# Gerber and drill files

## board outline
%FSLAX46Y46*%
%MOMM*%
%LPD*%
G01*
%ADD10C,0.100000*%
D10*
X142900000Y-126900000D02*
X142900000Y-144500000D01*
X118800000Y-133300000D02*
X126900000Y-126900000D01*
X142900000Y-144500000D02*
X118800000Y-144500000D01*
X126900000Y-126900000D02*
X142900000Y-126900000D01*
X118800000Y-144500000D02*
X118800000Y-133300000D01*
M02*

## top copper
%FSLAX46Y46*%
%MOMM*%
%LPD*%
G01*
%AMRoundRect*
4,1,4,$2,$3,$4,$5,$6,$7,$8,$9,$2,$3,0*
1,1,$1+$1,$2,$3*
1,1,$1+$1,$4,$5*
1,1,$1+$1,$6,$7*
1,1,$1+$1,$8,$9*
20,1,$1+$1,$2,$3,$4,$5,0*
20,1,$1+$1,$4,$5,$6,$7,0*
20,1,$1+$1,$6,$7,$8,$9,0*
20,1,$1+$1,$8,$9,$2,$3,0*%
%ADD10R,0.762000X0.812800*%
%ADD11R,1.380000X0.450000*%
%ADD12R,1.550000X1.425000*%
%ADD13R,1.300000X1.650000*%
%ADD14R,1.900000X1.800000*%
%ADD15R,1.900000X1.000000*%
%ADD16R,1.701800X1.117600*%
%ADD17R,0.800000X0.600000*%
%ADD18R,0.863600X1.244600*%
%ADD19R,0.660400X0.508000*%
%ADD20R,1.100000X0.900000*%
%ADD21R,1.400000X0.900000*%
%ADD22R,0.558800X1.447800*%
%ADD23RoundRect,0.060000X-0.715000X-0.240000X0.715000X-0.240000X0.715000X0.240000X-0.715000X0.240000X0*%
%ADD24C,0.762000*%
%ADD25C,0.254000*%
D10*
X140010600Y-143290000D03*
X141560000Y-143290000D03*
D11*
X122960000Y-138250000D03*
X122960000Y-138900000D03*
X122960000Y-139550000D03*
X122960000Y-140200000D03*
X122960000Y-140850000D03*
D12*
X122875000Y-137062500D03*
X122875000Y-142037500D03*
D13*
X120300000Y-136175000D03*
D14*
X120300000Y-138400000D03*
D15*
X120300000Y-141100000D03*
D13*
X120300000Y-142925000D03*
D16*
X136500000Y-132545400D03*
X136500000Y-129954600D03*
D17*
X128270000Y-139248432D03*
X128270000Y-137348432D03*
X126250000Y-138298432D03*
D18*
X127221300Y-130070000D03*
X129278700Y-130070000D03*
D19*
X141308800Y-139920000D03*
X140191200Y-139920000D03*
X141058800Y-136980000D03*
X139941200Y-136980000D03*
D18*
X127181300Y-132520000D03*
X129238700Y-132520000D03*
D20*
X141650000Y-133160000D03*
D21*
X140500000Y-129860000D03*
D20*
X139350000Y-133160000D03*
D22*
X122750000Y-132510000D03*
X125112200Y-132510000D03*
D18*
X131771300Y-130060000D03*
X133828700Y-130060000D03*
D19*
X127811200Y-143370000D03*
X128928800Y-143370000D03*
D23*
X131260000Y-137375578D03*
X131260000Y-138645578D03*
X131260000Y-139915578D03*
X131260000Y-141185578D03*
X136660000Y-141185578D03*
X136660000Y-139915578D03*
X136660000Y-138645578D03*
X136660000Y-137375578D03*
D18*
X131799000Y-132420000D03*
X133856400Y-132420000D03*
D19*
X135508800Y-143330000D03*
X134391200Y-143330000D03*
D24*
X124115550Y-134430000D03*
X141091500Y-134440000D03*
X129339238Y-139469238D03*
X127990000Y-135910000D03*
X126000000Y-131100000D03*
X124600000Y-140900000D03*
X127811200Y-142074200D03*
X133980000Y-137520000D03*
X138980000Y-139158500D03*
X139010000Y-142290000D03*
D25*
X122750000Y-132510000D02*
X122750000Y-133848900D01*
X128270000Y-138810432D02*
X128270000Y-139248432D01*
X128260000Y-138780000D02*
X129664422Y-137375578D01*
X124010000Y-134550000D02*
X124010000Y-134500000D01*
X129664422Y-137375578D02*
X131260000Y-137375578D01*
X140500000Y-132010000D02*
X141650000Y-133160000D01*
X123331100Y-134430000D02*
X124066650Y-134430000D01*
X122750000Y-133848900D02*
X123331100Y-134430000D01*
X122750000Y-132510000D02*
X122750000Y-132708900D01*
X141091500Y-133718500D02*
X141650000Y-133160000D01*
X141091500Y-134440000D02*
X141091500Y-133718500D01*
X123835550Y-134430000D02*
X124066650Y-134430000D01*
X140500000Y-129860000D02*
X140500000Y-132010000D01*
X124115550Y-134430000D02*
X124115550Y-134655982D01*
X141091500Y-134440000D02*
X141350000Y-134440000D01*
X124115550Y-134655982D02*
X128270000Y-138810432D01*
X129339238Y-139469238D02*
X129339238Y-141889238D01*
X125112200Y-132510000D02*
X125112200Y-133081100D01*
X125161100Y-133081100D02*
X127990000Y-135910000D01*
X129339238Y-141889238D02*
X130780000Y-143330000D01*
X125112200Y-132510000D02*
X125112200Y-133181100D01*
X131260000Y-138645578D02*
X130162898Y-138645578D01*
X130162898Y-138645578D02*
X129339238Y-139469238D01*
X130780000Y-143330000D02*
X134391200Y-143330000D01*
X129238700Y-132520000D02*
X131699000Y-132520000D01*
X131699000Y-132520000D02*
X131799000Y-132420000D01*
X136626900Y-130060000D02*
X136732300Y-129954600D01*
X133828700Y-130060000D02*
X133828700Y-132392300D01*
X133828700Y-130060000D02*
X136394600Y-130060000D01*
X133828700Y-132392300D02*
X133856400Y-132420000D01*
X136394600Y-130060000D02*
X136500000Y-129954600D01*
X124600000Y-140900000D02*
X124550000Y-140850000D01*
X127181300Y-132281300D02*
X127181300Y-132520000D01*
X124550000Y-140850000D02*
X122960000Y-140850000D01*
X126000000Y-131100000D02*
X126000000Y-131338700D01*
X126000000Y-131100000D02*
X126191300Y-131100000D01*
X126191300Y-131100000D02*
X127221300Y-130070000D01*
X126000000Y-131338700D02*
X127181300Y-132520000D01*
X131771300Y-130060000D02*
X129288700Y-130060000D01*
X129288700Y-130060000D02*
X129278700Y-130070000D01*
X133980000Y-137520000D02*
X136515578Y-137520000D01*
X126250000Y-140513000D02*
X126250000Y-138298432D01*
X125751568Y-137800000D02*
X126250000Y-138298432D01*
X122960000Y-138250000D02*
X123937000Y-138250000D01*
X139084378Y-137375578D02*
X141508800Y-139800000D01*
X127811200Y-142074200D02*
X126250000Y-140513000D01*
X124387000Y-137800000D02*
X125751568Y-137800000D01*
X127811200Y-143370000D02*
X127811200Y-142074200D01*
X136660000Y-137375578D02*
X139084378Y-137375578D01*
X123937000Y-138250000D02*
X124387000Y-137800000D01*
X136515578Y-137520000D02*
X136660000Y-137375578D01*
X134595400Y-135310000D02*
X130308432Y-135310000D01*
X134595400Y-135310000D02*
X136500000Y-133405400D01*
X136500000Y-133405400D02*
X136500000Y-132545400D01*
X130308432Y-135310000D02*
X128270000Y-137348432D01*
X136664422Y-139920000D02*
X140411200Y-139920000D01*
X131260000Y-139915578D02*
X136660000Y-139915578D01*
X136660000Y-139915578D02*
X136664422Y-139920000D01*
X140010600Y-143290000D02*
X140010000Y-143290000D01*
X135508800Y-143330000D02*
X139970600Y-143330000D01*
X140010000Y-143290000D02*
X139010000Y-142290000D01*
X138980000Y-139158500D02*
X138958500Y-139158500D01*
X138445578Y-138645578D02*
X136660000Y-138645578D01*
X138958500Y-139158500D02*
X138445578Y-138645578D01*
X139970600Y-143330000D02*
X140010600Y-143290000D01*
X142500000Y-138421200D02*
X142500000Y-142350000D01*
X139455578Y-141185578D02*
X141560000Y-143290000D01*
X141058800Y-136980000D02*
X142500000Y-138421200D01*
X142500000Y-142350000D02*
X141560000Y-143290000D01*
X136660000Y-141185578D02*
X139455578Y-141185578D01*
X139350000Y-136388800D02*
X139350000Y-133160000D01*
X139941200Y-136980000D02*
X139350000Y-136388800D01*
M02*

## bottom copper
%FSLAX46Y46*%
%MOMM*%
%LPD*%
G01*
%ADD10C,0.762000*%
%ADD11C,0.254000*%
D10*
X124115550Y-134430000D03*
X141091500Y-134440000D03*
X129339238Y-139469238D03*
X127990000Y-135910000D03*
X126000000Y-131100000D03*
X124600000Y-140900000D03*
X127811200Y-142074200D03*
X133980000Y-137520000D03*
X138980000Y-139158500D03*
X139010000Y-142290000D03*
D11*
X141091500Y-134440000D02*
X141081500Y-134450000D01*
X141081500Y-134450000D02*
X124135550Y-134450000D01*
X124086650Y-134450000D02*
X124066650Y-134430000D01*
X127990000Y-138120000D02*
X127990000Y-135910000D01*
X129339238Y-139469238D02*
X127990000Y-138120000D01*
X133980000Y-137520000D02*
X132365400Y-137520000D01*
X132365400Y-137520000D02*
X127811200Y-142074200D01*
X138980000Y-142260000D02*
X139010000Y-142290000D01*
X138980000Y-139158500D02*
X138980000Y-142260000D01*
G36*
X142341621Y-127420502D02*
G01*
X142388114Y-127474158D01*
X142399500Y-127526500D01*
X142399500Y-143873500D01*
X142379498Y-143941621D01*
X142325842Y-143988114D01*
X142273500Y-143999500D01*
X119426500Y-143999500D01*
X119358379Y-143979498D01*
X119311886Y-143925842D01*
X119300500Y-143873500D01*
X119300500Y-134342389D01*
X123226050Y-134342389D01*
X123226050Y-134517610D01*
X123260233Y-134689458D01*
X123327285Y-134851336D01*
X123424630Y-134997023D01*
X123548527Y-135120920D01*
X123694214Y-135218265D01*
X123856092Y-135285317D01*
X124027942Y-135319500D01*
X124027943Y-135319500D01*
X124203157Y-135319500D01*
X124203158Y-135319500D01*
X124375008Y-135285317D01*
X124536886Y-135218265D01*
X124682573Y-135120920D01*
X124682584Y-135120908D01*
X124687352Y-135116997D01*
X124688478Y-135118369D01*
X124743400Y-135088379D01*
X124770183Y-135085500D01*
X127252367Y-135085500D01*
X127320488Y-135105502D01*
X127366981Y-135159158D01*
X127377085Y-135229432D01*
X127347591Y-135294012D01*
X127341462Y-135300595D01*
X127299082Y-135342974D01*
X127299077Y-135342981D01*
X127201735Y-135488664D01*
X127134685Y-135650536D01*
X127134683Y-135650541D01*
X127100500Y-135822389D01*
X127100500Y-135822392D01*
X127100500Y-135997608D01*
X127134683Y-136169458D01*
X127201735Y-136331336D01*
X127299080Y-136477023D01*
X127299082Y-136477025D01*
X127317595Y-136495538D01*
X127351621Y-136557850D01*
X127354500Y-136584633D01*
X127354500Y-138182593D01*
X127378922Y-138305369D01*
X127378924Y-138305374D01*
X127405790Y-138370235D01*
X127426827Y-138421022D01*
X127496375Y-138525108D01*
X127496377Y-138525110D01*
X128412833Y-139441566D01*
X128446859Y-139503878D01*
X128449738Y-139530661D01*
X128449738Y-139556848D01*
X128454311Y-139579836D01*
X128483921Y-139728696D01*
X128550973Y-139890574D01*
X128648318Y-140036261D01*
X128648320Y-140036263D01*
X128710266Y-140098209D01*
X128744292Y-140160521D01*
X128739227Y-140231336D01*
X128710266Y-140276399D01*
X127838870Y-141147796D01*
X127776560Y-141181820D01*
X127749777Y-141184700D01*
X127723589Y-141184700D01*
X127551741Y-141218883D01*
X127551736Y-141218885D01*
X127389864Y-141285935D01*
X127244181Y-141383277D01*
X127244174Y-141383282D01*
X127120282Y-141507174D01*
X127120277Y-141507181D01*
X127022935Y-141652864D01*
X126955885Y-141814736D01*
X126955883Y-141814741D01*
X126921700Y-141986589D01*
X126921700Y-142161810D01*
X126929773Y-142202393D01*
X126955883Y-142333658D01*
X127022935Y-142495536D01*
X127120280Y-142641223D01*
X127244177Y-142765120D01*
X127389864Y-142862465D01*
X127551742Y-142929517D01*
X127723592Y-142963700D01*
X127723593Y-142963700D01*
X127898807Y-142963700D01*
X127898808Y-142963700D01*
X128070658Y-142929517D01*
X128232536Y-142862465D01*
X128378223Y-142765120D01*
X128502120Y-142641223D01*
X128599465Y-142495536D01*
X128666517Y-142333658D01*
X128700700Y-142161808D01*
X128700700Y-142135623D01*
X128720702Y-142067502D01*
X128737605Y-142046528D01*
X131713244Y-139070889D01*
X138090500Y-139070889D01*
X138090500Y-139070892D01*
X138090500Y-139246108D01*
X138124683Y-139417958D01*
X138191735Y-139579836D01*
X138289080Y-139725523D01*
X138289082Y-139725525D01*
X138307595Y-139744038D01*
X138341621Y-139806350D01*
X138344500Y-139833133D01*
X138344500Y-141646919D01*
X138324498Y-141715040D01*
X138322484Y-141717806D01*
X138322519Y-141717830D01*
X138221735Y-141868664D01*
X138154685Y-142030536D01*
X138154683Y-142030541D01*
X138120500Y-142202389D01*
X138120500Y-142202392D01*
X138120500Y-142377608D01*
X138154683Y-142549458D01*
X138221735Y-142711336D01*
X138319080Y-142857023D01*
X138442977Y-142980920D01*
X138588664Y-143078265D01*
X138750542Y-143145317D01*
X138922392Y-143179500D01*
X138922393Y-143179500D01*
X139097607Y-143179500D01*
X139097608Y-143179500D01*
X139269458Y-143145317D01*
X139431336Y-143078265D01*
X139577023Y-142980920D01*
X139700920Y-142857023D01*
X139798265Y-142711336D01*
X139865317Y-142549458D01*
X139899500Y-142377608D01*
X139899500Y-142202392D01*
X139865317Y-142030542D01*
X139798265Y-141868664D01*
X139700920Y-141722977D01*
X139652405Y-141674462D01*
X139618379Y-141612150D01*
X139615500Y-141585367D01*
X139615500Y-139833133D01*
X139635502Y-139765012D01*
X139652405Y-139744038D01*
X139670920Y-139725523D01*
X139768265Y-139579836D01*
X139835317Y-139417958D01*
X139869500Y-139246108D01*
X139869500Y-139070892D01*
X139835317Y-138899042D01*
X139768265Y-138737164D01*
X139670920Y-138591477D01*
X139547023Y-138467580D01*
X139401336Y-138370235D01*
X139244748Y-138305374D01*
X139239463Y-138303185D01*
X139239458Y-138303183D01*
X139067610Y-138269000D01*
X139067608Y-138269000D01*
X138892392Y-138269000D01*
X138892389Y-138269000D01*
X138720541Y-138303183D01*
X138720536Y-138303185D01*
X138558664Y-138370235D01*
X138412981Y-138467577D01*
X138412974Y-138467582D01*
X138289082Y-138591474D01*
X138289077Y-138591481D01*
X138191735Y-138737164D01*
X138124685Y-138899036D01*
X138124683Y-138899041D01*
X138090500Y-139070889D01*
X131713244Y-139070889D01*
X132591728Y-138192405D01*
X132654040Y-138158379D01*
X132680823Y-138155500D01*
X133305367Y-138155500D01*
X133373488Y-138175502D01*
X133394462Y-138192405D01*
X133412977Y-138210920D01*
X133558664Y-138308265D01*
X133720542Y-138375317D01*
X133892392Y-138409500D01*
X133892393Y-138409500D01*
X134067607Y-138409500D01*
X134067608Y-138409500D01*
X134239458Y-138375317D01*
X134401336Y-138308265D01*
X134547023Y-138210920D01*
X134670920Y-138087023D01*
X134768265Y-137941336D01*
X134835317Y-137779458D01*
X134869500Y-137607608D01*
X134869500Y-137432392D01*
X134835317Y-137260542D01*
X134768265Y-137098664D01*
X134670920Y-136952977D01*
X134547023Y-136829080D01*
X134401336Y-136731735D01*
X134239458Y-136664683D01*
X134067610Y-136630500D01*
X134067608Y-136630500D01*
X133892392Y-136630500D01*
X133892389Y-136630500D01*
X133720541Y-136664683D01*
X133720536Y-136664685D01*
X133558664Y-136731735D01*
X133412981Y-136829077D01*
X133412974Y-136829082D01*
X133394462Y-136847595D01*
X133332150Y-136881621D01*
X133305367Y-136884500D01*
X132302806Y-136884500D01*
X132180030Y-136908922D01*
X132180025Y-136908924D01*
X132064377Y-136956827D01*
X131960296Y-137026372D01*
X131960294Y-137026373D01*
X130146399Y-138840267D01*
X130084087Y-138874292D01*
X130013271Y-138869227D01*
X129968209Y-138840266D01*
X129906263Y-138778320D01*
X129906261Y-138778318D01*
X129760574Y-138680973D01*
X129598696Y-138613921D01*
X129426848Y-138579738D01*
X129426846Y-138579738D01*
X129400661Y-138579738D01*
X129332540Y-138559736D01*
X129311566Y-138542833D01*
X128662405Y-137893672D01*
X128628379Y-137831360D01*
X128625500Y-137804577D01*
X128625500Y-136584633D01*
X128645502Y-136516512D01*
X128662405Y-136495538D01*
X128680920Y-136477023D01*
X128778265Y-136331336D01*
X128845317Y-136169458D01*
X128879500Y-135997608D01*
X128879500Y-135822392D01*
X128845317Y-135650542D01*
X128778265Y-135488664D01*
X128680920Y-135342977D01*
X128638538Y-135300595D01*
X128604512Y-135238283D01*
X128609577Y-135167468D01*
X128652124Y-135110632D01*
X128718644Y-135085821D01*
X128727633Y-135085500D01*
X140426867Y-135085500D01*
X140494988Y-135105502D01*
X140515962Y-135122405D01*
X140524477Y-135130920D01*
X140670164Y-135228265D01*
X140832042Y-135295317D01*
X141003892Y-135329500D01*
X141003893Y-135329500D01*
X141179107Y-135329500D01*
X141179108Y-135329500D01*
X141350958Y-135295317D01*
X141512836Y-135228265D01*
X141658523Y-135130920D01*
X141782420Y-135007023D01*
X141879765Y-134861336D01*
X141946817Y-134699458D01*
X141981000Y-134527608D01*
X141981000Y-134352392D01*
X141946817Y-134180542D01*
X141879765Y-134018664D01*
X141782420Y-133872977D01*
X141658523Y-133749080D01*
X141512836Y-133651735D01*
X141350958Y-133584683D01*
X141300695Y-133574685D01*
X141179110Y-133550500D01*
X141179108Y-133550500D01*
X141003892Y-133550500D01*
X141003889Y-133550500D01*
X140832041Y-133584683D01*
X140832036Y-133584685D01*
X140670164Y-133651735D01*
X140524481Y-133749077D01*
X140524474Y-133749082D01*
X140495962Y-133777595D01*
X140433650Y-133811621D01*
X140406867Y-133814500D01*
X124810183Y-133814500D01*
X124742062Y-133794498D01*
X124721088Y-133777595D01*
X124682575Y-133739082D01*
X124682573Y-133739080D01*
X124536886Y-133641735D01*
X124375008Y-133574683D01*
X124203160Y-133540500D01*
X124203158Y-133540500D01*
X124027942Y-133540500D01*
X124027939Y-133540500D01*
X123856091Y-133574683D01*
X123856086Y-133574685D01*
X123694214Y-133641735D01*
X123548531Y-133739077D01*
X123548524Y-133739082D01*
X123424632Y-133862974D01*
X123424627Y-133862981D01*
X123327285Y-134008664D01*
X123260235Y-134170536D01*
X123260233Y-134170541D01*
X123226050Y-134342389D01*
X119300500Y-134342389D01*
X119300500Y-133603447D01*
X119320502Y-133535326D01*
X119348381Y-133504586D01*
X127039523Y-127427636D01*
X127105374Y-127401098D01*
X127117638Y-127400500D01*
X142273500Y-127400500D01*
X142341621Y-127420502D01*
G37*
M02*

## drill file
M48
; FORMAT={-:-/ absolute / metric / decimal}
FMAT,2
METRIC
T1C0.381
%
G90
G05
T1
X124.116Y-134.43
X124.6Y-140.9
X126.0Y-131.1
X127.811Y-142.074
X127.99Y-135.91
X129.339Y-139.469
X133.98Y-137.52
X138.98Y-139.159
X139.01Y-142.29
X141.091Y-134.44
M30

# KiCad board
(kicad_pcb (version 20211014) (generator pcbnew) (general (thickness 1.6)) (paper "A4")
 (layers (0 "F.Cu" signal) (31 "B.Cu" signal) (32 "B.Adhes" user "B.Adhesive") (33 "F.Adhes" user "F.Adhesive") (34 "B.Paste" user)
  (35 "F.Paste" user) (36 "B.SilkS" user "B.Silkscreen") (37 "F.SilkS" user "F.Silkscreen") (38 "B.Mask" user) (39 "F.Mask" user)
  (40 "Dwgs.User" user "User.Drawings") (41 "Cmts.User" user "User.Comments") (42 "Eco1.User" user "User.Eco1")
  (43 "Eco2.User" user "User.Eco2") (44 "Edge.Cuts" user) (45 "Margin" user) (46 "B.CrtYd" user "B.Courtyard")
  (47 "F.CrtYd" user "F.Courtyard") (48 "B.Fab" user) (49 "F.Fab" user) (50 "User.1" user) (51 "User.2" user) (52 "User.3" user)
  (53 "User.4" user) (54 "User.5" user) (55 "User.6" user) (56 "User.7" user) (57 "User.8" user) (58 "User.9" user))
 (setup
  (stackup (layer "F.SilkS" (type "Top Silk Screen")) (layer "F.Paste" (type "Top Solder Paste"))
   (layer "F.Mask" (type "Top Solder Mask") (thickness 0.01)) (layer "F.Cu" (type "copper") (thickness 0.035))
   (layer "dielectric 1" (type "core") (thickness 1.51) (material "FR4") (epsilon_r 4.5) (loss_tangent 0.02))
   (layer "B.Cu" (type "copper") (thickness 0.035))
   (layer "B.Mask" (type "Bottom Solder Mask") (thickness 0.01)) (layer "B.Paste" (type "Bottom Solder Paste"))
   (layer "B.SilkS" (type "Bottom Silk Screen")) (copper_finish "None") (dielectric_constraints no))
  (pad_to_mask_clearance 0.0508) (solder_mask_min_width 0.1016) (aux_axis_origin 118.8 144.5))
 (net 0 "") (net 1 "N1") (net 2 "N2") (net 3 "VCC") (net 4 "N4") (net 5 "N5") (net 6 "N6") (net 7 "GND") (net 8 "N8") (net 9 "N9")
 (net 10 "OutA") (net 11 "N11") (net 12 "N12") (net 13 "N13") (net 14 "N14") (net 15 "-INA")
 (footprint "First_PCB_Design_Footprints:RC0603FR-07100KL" (layer "F.Cu") (at 140.7853 143.29)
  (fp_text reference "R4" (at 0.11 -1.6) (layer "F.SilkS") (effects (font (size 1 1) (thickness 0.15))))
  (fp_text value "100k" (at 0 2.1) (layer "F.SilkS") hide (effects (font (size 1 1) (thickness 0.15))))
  (pad "1" smd rect (at -0.7747 0) (size 0.762 0.8128) (layers "F.Cu" "F.Paste" "F.Mask") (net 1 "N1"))
  (pad "2" smd rect (at 0.7747 0) (size 0.762 0.8128) (layers "F.Cu" "F.Paste" "F.Mask") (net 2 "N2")))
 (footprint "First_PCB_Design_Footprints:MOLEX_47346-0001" (layer "F.Cu") (at 120.3 139.55 -90)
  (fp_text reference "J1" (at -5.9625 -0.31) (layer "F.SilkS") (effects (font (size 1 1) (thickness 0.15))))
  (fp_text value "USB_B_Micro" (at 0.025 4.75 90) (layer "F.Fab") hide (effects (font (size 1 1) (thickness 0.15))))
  (pad "1" smd rect (at -1.3 -2.66 270) (size 0.45 1.38) (layers "F.Cu" "F.Paste" "F.Mask") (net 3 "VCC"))
  (pad "2" smd rect (at -0.65 -2.66 270) (size 0.45 1.38) (layers "F.Cu" "F.Paste" "F.Mask") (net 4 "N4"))
  (pad "3" smd rect (at 0 -2.66 270) (size 0.45 1.38) (layers "F.Cu" "F.Paste" "F.Mask") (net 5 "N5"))
  (pad "4" smd rect (at 0.65 -2.66 270) (size 0.45 1.38) (layers "F.Cu" "F.Paste" "F.Mask") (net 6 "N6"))
  (pad "5" smd rect (at 1.3 -2.66 270) (size 0.45 1.38) (layers "F.Cu" "F.Paste" "F.Mask") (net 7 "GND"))
  (pad "S1" smd rect (at -2.4875 -2.575 270) (size 1.425 1.55) (layers "F.Cu" "F.Paste" "F.Mask"))
  (pad "S2" smd rect (at 2.4875 -2.575 270) (size 1.425 1.55) (layers "F.Cu" "F.Paste" "F.Mask"))
  (pad "S3" smd rect (at -3.375 0 270) (size 1.65 1.3) (layers "F.Cu" "F.Paste" "F.Mask"))
  (pad "S4" smd rect (at -1.15 0 270) (size 1.8 1.9) (layers "F.Cu" "F.Paste" "F.Mask"))
  (pad "S5" smd rect (at 1.55 0 270) (size 1 1.9) (layers "F.Cu" "F.Paste" "F.Mask"))
  (pad "S6" smd rect (at 3.375 0 270) (size 1.65 1.3) (layers "F.Cu" "F.Paste" "F.Mask")))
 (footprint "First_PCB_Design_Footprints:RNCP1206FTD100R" (layer "F.Cu") (at 136.5 131.25 90)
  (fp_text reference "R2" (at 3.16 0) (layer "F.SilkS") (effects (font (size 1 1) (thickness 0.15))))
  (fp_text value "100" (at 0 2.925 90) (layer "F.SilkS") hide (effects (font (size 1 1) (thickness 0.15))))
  (pad "1" smd rect (at -1.2954 0 90) (size 1.1176 1.7018) (layers "F.Cu" "F.Paste" "F.Mask") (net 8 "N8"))
  (pad "2" smd rect (at 1.2954 0 90) (size 1.1176 1.7018) (layers "F.Cu" "F.Paste" "F.Mask") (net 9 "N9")))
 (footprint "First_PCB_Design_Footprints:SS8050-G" (layer "F.Cu") (at 127.26 138.298432 90)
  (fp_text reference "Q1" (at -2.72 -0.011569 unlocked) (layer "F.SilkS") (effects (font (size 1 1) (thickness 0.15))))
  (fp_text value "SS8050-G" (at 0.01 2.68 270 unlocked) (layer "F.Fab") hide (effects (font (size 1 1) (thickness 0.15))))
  (pad "1" smd rect (at -0.95 1.01 90) (size 0.6 0.8) (layers "F.Cu" "F.Mask") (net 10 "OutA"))
  (pad "2" smd rect (at 0.95 1.01 90) (size 0.6 0.8) (layers "F.Cu" "F.Mask") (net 8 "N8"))
  (pad "3" smd rect (at 0 -1.01 90) (size 0.6 0.8) (layers "F.Cu" "F.Mask") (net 3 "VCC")))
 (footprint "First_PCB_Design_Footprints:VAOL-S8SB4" (layer "F.Cu") (at 128.25 130.07)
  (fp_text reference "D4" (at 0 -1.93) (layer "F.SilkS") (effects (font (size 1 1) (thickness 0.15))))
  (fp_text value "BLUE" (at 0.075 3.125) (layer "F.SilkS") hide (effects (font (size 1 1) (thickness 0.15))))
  (pad "1" smd rect (at -1.0287 0) (size 0.8636 1.2446) (layers "F.Cu" "F.Paste" "F.Mask") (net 7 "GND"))
  (pad "2" smd rect (at 1.0287 0) (size 0.8636 1.2446) (layers "F.Cu" "F.Paste" "F.Mask") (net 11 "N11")))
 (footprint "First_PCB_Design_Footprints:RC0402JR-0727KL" (layer "F.Cu") (at 140.75 139.92 180)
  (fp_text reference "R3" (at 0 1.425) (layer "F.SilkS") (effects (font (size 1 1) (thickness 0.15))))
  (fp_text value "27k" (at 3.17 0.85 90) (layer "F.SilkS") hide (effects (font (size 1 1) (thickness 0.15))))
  (pad "1" smd rect (at -0.5588 0 180) (size 0.6604 0.508) (layers "F.Cu" "F.Paste" "F.Mask") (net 3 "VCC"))
  (pad "2" smd rect (at 0.5588 0 180) (size 0.6604 0.508) (layers "F.Cu" "F.Paste" "F.Mask") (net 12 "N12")))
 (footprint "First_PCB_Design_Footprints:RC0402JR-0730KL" (layer "F.Cu") (at 140.5 136.98 180)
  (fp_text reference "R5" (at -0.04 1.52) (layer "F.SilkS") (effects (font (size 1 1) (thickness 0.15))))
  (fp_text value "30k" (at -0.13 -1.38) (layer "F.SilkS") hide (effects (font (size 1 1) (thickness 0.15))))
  (pad "1" smd rect (at -0.5588 0 180) (size 0.6604 0.508) (layers "F.Cu" "F.Paste" "F.Mask") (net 2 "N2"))
  (pad "2" smd rect (at 0.5588 0 180) (size 0.6604 0.508) (layers "F.Cu" "F.Paste" "F.Mask") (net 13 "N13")))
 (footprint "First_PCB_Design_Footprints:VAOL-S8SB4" (layer "F.Cu") (at 128.21 132.52)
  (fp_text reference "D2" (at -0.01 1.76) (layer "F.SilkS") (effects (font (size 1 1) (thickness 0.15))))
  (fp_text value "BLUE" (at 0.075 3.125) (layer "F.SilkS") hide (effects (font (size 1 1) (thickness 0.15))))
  (pad "1" smd rect (at -1.0287 0) (size 0.8636 1.2446) (layers "F.Cu" "F.Paste" "F.Mask") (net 7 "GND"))
  (pad "2" smd rect (at 1.0287 0) (size 0.8636 1.2446) (layers "F.Cu" "F.Paste" "F.Mask") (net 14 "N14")))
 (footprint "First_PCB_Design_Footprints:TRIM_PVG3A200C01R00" (layer "F.Cu") (at 140.5 131.51)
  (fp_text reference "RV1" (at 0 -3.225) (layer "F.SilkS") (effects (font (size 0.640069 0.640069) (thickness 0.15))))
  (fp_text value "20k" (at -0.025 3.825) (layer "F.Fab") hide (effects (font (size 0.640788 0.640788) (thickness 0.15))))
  (pad "1" smd rect (at 1.15 1.65) (size 1.1 0.9) (layers "F.Cu" "F.Paste" "F.Mask") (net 10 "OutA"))
  (pad "2" smd rect (at 0 -1.65) (size 1.4 0.9) (layers "F.Cu" "F.Paste" "F.Mask") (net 10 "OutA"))
  (pad "3" smd rect (at -1.15 1.65) (size 1.1 0.9) (layers "F.Cu" "F.Paste" "F.Mask") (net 13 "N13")))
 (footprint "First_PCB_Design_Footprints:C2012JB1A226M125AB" (layer "F.Cu") (at 123.9311 132.51)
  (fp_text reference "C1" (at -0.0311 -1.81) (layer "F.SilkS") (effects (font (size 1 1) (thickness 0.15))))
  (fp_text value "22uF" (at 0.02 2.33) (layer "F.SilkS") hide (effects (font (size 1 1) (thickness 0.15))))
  (pad "1" smd rect (at -1.1811 0) (size 0.5588 1.4478) (layers "F.Cu" "F.Paste" "F.Mask") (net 10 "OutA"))
  (pad "2" smd rect (at 1.1811 0) (size 0.5588 1.4478) (layers "F.Cu" "F.Paste" "F.Mask") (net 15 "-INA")))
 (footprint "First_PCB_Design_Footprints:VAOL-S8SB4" (layer "F.Cu") (at 132.8 130.06)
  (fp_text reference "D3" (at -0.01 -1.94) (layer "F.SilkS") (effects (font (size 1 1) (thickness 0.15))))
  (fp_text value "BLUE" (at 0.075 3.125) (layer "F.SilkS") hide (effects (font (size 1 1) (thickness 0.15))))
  (pad "1" smd rect (at -1.0287 0) (size 0.8636 1.2446) (layers "F.Cu" "F.Paste" "F.Mask") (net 11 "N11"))
  (pad "2" smd rect (at 1.0287 0) (size 0.8636 1.2446) (layers "F.Cu" "F.Paste" "F.Mask") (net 9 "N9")))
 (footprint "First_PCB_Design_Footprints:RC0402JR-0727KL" (layer "F.Cu") (at 128.37 143.37)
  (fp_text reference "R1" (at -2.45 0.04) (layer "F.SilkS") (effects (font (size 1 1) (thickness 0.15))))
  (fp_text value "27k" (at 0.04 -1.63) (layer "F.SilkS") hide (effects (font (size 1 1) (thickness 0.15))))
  (pad "1" smd rect (at -0.5588 0) (size 0.6604 0.508) (layers "F.Cu" "F.Paste" "F.Mask") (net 3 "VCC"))
  (pad "2" smd rect (at 0.5588 0) (size 0.6604 0.508) (layers "F.Cu" "F.Paste" "F.Mask") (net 7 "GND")))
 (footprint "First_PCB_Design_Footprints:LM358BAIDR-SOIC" (layer "F.Cu") (at 133.96 139.280578)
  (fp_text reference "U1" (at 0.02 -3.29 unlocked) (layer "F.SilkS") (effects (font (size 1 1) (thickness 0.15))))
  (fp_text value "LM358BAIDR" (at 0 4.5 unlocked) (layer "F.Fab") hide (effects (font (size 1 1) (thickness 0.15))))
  (pad "1" smd roundrect (at -2.7 -1.905) (size 1.55 0.6) (layers "F.Cu" "F.Mask") (roundrect_rratio 0.1) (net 10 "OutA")
   (solder_mask_margin 0.07))
  (pad "2" smd roundrect (at -2.7 -0.635) (size 1.55 0.6) (layers "F.Cu" "F.Mask") (roundrect_rratio 0.1) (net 15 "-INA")
   (solder_mask_margin 0.07))
  (pad "3" smd roundrect (at -2.7 0.635) (size 1.55 0.6) (layers "F.Cu" "F.Mask") (roundrect_rratio 0.1) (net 12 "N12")
   (solder_mask_margin 0.07))
  (pad "4" smd roundrect (at -2.7 1.905) (size 1.55 0.6) (layers "F.Cu" "F.Mask") (roundrect_rratio 0.1) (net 7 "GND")
   (solder_mask_margin 0.07))
  (pad "5" smd roundrect (at 2.7 1.905) (size 1.55 0.6) (layers "F.Cu" "F.Mask") (roundrect_rratio 0.1) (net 2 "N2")
   (solder_mask_margin 0.07))
  (pad "6" smd roundrect (at 2.7 0.635) (size 1.55 0.6) (layers "F.Cu" "F.Mask") (roundrect_rratio 0.1) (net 12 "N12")
   (solder_mask_margin 0.07))
  (pad "7" smd roundrect (at 2.7 -0.635) (size 1.55 0.6) (layers "F.Cu" "F.Mask") (roundrect_rratio 0.1) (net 1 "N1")
   (solder_mask_margin 0.07))
  (pad "8" smd roundrect (at 2.7 -1.905) (size 1.55 0.6) (layers "F.Cu" "F.Mask") (roundrect_rratio 0.1) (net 3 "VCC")
   (solder_mask_margin 0.07)))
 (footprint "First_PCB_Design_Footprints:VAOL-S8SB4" (layer "F.Cu") (at 132.8277 132.42)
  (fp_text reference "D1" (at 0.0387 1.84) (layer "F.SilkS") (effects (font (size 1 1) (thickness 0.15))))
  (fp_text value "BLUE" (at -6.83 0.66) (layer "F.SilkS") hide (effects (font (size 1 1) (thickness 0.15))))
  (pad "1" smd rect (at -1.0287 0) (size 0.8636 1.2446) (layers "F.Cu" "F.Paste" "F.Mask") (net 14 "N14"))
  (pad "2" smd rect (at 1.0287 0) (size 0.8636 1.2446) (layers "F.Cu" "F.Paste" "F.Mask") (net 9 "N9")))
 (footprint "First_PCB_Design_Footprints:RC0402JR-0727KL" (layer "F.Cu") (at 134.95 143.33 180)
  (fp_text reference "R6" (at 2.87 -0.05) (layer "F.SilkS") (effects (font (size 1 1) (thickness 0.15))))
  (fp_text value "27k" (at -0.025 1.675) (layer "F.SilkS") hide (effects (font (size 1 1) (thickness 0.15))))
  (pad "1" smd rect (at -0.5588 0 180) (size 0.6604 0.508) (layers "F.Cu" "F.Paste" "F.Mask") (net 1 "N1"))
  (pad "2" smd rect (at 0.5588 0 180) (size 0.6604 0.508) (layers "F.Cu" "F.Paste" "F.Mask") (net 15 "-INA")))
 (gr_line (start 142.9 126.9) (end 142.9 144.5) (layer "Edge.Cuts") (width 0.1))
 (gr_line (start 118.8 133.3) (end 126.9 126.9) (layer "Edge.Cuts") (width 0.1))
 (gr_line (start 142.9 144.5) (end 118.8 144.5) (layer "Edge.Cuts") (width 0.1))
 (gr_line (start 126.9 126.9) (end 142.9 126.9) (layer "Edge.Cuts") (width 0.1))
 (gr_line (start 118.8 144.5) (end 118.8 133.3) (layer "Edge.Cuts") (width 0.1))
 (segment (start 122.75 132.51) (end 122.75 133.8489) (width 0.254) (layer "F.Cu") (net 10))
 (segment (start 128.27 138.810432) (end 128.27 139.248432) (width 0.254) (layer "F.Cu") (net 10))
 (segment (start 128.26 138.78) (end 129.664422 137.375578) (width 0.254) (layer "F.Cu") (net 10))
 (segment (start 124.01 134.55) (end 124.01 134.5) (width 0.254) (layer "F.Cu") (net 10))
 (segment (start 129.664422 137.375578) (end 131.26 137.375578) (width 0.254) (layer "F.Cu") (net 10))
 (segment (start 140.5 132.01) (end 141.65 133.16) (width 0.254) (layer "F.Cu") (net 10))
 (segment (start 123.3311 134.43) (end 124.06665 134.43) (width 0.254) (layer "F.Cu") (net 10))
 (segment (start 122.75 133.8489) (end 123.3311 134.43) (width 0.254) (layer "F.Cu") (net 10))
 (segment (start 122.75 132.51) (end 122.75 132.7089) (width 0.254) (layer "F.Cu") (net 10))
 (segment (start 141.0915 133.7185) (end 141.65 133.16) (width 0.254) (layer "F.Cu") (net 10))
 (segment (start 141.0915 134.44) (end 141.0915 133.7185) (width 0.254) (layer "F.Cu") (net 10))
 (segment (start 123.83555 134.43) (end 124.06665 134.43) (width 0.254) (layer "F.Cu") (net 10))
 (segment (start 140.5 129.86) (end 140.5 132.01) (width 0.254) (layer "F.Cu") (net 10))
 (segment (start 124.11555 134.43) (end 124.11555 134.655982) (width 0.254) (layer "F.Cu") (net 10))
 (segment (start 141.0915 134.44) (end 141.35 134.44) (width 0.254) (layer "F.Cu") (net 10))
 (segment (start 124.11555 134.655982) (end 128.27 138.810432) (width 0.254) (layer "F.Cu") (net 10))
 (via (at 124.11555 134.43) (size 0.762) (drill 0.381) (layers "F.Cu" "B.Cu") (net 10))
 (via (at 141.0915 134.44) (size 0.762) (drill 0.381) (layers "F.Cu" "B.Cu") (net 10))
 (segment (start 141.0915 134.44) (end 141.0815 134.45) (width 0.254) (layer "B.Cu") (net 10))
 (segment (start 141.0815 134.45) (end 124.13555 134.45) (width 0.254) (layer "B.Cu") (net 10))
 (segment (start 124.08665 134.45) (end 124.06665 134.43) (width 0.254) (layer "B.Cu") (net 10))
 (segment (start 129.339238 139.469238) (end 129.339238 141.889238) (width 0.254) (layer "F.Cu") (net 15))
 (segment (start 125.1122 132.51) (end 125.1122 133.0811) (width 0.254) (layer "F.Cu") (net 15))
 (segment (start 125.1611 133.0811) (end 127.99 135.91) (width 0.254) (layer "F.Cu") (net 15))
 (segment (start 129.339238 141.889238) (end 130.78 143.33) (width 0.254) (layer "F.Cu") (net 15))
 (segment (start 125.1122 132.51) (end 125.1122 133.1811) (width 0.254) (layer "F.Cu") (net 15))
 (segment (start 131.26 138.645578) (end 130.162898 138.645578) (width 0.254) (layer "F.Cu") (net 15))
 (segment (start 130.162898 138.645578) (end 129.339238 139.469238) (width 0.254) (layer "F.Cu") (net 15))
 (segment (start 130.78 143.33) (end 134.3912 143.33) (width 0.254) (layer "F.Cu") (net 15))
 (via (at 129.339238 139.469238) (size 0.762) (drill 0.381) (layers "F.Cu" "B.Cu") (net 15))
 (via (at 127.99 135.91) (size 0.762) (drill 0.381) (layers "F.Cu" "B.Cu") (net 15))
 (segment (start 127.99 138.12) (end 127.99 135.91) (width 0.254) (layer "B.Cu") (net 15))
 (segment (start 129.339238 139.469238) (end 127.99 138.12) (width 0.254) (layer "B.Cu") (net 15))
 (segment (start 129.2387 132.52) (end 131.699 132.52) (width 0.254) (layer "F.Cu") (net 14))
 (segment (start 131.699 132.52) (end 131.799 132.42) (width 0.254) (layer "F.Cu") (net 14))
 (segment (start 136.6269 130.06) (end 136.7323 129.9546) (width 0.254) (layer "F.Cu") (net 9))
 (segment (start 133.8287 130.06) (end 133.8287 132.3923) (width 0.254) (layer "F.Cu") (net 9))
 (segment (start 133.8287 130.06) (end 136.3946 130.06) (width 0.254) (layer "F.Cu") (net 9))
 (segment (start 133.8287 132.3923) (end 133.8564 132.42) (width 0.254) (layer "F.Cu") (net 9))
 (segment (start 136.3946 130.06) (end 136.5 129.9546) (width 0.254) (layer "F.Cu") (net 9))
 (segment (start 124.6 140.9) (end 124.55 140.85) (width 0.254) (layer "F.Cu") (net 7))
 (segment (start 127.1813 132.2813) (end 127.1813 132.52) (width 0.254) (layer "F.Cu") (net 7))
 (segment (start 124.55 140.85) (end 122.96 140.85) (width 0.254) (layer "F.Cu") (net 7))
 (segment (start 126 131.1) (end 126 131.3387) (width 0.254) (layer "F.Cu") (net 7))
 (segment (start 126 131.1) (end 126.1913 131.1) (width 0.254) (layer "F.Cu") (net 7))
 (segment (start 126.1913 131.1) (end 127.2213 130.07) (width 0.254) (layer "F.Cu") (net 7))
 (segment (start 126 131.3387) (end 127.1813 132.52) (width 0.254) (layer "F.Cu") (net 7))
 (via (at 126 131.1) (size 0.762) (drill 0.381) (layers "F.Cu" "B.Cu") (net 7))
 (via (at 124.6 140.9) (size 0.762) (drill 0.381) (layers "F.Cu" "B.Cu") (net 7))
 (segment (start 131.7713 130.06) (end 129.2887 130.06) (width 0.254) (layer "F.Cu") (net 11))
 (segment (start 129.2887 130.06) (end 129.2787 130.07) (width 0.254) (layer "F.Cu") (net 11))
 (segment (start 133.98 137.52) (end 136.515578 137.52) (width 0.254) (layer "F.Cu") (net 3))
 (segment (start 126.25 140.513) (end 126.25 138.298432) (width 0.254) (layer "F.Cu") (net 3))
 (segment (start 125.751568 137.8) (end 126.25 138.298432) (width 0.254) (layer "F.Cu") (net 3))
 (segment (start 122.96 138.25) (end 123.937 138.25) (width 0.254) (layer "F.Cu") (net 3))
 (segment (start 139.084378 137.375578) (end 141.5088 139.8) (width 0.254) (layer "F.Cu") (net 3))
 (segment (start 127.8112 142.0742) (end 126.25 140.513) (width 0.254) (layer "F.Cu") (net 3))
 (segment (start 124.387 137.8) (end 125.751568 137.8) (width 0.254) (layer "F.Cu") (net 3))
 (segment (start 127.8112 143.37) (end 127.8112 142.0742) (width 0.254) (layer "F.Cu") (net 3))
 (segment (start 136.66 137.375578) (end 139.084378 137.375578) (width 0.254) (layer "F.Cu") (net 3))
 (segment (start 123.937 138.25) (end 124.387 137.8) (width 0.254) (layer "F.Cu") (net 3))
 (segment (start 136.515578 137.52) (end 136.66 137.375578) (width 0.254) (layer "F.Cu") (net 3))
 (via (at 127.8112 142.0742) (size 0.762) (drill 0.381) (layers "F.Cu" "B.Cu") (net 3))
 (via (at 133.98 137.52) (size 0.762) (drill 0.381) (layers "F.Cu" "B.Cu") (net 3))
 (segment (start 133.98 137.52) (end 132.3654 137.52) (width 0.254) (layer "B.Cu") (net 3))
 (segment (start 132.3654 137.52) (end 127.8112 142.0742) (width 0.254) (layer "B.Cu") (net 3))
 (segment (start 134.5954 135.31) (end 130.308432 135.31) (width 0.254) (layer "F.Cu") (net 8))
 (segment (start 134.5954 135.31) (end 136.5 133.4054) (width 0.254) (layer "F.Cu") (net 8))
 (segment (start 136.5 133.4054) (end 136.5 132.5454) (width 0.254) (layer "F.Cu") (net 8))
 (segment (start 130.308432 135.31) (end 128.27 137.348432) (width 0.254) (layer "F.Cu") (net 8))
 (segment (start 136.664422 139.92) (end 140.4112 139.92) (width 0.254) (layer "F.Cu") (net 12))
 (segment (start 131.26 139.915578) (end 136.66 139.915578) (width 0.254) (layer "F.Cu") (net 12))
 (segment (start 136.66 139.915578) (end 136.664422 139.92) (width 0.254) (layer "F.Cu") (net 12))
 (segment (start 140.0106 143.29) (end 140.01 143.29) (width 0.254) (layer "F.Cu") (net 1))
 (segment (start 135.5088 143.33) (end 139.9706 143.33) (width 0.254) (layer "F.Cu") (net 1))
 (segment (start 140.01 143.29) (end 139.01 142.29) (width 0.254) (layer "F.Cu") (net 1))
 (segment (start 138.98 139.1585) (end 138.9585 139.1585) (width 0.254) (layer "F.Cu") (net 1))
 (segment (start 138.445578 138.645578) (end 136.66 138.645578) (width 0.254) (layer "F.Cu") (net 1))
 (segment (start 138.9585 139.1585) (end 138.445578 138.645578) (width 0.254) (layer "F.Cu") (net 1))
 (segment (start 139.9706 143.33) (end 140.0106 143.29) (width 0.254) (layer "F.Cu") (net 1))
 (via (at 138.98 139.1585) (size 0.762) (drill 0.381) (layers "F.Cu" "B.Cu") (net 1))
 (via (at 139.01 142.29) (size 0.762) (drill 0.381) (layers "F.Cu" "B.Cu") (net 1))
 (segment (start 138.98 142.26) (end 139.01 142.29) (width 0.254) (layer "B.Cu") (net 1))
 (segment (start 138.98 139.1585) (end 138.98 142.26) (width 0.254) (layer "B.Cu") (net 1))
 (segment (start 142.5 138.4212) (end 142.5 142.35) (width 0.254) (layer "F.Cu") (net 2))
 (segment (start 139.455578 141.185578) (end 141.56 143.29) (width 0.254) (layer "F.Cu") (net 2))
 (segment (start 141.0588 136.98) (end 142.5 138.4212) (width 0.254) (layer "F.Cu") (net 2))
 (segment (start 142.5 142.35) (end 141.56 143.29) (width 0.254) (layer "F.Cu") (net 2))
 (segment (start 136.66 141.185578) (end 139.455578 141.185578) (width 0.254) (layer "F.Cu") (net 2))
 (segment (start 139.35 136.3888) (end 139.35 133.16) (width 0.254) (layer "F.Cu") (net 13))
 (segment (start 139.9412 136.98) (end 139.35 136.3888) (width 0.254) (layer "F.Cu") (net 13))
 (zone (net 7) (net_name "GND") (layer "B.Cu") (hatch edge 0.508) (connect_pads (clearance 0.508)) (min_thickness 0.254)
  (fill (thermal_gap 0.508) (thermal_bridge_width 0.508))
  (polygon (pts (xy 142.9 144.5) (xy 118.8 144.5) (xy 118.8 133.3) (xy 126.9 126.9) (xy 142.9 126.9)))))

